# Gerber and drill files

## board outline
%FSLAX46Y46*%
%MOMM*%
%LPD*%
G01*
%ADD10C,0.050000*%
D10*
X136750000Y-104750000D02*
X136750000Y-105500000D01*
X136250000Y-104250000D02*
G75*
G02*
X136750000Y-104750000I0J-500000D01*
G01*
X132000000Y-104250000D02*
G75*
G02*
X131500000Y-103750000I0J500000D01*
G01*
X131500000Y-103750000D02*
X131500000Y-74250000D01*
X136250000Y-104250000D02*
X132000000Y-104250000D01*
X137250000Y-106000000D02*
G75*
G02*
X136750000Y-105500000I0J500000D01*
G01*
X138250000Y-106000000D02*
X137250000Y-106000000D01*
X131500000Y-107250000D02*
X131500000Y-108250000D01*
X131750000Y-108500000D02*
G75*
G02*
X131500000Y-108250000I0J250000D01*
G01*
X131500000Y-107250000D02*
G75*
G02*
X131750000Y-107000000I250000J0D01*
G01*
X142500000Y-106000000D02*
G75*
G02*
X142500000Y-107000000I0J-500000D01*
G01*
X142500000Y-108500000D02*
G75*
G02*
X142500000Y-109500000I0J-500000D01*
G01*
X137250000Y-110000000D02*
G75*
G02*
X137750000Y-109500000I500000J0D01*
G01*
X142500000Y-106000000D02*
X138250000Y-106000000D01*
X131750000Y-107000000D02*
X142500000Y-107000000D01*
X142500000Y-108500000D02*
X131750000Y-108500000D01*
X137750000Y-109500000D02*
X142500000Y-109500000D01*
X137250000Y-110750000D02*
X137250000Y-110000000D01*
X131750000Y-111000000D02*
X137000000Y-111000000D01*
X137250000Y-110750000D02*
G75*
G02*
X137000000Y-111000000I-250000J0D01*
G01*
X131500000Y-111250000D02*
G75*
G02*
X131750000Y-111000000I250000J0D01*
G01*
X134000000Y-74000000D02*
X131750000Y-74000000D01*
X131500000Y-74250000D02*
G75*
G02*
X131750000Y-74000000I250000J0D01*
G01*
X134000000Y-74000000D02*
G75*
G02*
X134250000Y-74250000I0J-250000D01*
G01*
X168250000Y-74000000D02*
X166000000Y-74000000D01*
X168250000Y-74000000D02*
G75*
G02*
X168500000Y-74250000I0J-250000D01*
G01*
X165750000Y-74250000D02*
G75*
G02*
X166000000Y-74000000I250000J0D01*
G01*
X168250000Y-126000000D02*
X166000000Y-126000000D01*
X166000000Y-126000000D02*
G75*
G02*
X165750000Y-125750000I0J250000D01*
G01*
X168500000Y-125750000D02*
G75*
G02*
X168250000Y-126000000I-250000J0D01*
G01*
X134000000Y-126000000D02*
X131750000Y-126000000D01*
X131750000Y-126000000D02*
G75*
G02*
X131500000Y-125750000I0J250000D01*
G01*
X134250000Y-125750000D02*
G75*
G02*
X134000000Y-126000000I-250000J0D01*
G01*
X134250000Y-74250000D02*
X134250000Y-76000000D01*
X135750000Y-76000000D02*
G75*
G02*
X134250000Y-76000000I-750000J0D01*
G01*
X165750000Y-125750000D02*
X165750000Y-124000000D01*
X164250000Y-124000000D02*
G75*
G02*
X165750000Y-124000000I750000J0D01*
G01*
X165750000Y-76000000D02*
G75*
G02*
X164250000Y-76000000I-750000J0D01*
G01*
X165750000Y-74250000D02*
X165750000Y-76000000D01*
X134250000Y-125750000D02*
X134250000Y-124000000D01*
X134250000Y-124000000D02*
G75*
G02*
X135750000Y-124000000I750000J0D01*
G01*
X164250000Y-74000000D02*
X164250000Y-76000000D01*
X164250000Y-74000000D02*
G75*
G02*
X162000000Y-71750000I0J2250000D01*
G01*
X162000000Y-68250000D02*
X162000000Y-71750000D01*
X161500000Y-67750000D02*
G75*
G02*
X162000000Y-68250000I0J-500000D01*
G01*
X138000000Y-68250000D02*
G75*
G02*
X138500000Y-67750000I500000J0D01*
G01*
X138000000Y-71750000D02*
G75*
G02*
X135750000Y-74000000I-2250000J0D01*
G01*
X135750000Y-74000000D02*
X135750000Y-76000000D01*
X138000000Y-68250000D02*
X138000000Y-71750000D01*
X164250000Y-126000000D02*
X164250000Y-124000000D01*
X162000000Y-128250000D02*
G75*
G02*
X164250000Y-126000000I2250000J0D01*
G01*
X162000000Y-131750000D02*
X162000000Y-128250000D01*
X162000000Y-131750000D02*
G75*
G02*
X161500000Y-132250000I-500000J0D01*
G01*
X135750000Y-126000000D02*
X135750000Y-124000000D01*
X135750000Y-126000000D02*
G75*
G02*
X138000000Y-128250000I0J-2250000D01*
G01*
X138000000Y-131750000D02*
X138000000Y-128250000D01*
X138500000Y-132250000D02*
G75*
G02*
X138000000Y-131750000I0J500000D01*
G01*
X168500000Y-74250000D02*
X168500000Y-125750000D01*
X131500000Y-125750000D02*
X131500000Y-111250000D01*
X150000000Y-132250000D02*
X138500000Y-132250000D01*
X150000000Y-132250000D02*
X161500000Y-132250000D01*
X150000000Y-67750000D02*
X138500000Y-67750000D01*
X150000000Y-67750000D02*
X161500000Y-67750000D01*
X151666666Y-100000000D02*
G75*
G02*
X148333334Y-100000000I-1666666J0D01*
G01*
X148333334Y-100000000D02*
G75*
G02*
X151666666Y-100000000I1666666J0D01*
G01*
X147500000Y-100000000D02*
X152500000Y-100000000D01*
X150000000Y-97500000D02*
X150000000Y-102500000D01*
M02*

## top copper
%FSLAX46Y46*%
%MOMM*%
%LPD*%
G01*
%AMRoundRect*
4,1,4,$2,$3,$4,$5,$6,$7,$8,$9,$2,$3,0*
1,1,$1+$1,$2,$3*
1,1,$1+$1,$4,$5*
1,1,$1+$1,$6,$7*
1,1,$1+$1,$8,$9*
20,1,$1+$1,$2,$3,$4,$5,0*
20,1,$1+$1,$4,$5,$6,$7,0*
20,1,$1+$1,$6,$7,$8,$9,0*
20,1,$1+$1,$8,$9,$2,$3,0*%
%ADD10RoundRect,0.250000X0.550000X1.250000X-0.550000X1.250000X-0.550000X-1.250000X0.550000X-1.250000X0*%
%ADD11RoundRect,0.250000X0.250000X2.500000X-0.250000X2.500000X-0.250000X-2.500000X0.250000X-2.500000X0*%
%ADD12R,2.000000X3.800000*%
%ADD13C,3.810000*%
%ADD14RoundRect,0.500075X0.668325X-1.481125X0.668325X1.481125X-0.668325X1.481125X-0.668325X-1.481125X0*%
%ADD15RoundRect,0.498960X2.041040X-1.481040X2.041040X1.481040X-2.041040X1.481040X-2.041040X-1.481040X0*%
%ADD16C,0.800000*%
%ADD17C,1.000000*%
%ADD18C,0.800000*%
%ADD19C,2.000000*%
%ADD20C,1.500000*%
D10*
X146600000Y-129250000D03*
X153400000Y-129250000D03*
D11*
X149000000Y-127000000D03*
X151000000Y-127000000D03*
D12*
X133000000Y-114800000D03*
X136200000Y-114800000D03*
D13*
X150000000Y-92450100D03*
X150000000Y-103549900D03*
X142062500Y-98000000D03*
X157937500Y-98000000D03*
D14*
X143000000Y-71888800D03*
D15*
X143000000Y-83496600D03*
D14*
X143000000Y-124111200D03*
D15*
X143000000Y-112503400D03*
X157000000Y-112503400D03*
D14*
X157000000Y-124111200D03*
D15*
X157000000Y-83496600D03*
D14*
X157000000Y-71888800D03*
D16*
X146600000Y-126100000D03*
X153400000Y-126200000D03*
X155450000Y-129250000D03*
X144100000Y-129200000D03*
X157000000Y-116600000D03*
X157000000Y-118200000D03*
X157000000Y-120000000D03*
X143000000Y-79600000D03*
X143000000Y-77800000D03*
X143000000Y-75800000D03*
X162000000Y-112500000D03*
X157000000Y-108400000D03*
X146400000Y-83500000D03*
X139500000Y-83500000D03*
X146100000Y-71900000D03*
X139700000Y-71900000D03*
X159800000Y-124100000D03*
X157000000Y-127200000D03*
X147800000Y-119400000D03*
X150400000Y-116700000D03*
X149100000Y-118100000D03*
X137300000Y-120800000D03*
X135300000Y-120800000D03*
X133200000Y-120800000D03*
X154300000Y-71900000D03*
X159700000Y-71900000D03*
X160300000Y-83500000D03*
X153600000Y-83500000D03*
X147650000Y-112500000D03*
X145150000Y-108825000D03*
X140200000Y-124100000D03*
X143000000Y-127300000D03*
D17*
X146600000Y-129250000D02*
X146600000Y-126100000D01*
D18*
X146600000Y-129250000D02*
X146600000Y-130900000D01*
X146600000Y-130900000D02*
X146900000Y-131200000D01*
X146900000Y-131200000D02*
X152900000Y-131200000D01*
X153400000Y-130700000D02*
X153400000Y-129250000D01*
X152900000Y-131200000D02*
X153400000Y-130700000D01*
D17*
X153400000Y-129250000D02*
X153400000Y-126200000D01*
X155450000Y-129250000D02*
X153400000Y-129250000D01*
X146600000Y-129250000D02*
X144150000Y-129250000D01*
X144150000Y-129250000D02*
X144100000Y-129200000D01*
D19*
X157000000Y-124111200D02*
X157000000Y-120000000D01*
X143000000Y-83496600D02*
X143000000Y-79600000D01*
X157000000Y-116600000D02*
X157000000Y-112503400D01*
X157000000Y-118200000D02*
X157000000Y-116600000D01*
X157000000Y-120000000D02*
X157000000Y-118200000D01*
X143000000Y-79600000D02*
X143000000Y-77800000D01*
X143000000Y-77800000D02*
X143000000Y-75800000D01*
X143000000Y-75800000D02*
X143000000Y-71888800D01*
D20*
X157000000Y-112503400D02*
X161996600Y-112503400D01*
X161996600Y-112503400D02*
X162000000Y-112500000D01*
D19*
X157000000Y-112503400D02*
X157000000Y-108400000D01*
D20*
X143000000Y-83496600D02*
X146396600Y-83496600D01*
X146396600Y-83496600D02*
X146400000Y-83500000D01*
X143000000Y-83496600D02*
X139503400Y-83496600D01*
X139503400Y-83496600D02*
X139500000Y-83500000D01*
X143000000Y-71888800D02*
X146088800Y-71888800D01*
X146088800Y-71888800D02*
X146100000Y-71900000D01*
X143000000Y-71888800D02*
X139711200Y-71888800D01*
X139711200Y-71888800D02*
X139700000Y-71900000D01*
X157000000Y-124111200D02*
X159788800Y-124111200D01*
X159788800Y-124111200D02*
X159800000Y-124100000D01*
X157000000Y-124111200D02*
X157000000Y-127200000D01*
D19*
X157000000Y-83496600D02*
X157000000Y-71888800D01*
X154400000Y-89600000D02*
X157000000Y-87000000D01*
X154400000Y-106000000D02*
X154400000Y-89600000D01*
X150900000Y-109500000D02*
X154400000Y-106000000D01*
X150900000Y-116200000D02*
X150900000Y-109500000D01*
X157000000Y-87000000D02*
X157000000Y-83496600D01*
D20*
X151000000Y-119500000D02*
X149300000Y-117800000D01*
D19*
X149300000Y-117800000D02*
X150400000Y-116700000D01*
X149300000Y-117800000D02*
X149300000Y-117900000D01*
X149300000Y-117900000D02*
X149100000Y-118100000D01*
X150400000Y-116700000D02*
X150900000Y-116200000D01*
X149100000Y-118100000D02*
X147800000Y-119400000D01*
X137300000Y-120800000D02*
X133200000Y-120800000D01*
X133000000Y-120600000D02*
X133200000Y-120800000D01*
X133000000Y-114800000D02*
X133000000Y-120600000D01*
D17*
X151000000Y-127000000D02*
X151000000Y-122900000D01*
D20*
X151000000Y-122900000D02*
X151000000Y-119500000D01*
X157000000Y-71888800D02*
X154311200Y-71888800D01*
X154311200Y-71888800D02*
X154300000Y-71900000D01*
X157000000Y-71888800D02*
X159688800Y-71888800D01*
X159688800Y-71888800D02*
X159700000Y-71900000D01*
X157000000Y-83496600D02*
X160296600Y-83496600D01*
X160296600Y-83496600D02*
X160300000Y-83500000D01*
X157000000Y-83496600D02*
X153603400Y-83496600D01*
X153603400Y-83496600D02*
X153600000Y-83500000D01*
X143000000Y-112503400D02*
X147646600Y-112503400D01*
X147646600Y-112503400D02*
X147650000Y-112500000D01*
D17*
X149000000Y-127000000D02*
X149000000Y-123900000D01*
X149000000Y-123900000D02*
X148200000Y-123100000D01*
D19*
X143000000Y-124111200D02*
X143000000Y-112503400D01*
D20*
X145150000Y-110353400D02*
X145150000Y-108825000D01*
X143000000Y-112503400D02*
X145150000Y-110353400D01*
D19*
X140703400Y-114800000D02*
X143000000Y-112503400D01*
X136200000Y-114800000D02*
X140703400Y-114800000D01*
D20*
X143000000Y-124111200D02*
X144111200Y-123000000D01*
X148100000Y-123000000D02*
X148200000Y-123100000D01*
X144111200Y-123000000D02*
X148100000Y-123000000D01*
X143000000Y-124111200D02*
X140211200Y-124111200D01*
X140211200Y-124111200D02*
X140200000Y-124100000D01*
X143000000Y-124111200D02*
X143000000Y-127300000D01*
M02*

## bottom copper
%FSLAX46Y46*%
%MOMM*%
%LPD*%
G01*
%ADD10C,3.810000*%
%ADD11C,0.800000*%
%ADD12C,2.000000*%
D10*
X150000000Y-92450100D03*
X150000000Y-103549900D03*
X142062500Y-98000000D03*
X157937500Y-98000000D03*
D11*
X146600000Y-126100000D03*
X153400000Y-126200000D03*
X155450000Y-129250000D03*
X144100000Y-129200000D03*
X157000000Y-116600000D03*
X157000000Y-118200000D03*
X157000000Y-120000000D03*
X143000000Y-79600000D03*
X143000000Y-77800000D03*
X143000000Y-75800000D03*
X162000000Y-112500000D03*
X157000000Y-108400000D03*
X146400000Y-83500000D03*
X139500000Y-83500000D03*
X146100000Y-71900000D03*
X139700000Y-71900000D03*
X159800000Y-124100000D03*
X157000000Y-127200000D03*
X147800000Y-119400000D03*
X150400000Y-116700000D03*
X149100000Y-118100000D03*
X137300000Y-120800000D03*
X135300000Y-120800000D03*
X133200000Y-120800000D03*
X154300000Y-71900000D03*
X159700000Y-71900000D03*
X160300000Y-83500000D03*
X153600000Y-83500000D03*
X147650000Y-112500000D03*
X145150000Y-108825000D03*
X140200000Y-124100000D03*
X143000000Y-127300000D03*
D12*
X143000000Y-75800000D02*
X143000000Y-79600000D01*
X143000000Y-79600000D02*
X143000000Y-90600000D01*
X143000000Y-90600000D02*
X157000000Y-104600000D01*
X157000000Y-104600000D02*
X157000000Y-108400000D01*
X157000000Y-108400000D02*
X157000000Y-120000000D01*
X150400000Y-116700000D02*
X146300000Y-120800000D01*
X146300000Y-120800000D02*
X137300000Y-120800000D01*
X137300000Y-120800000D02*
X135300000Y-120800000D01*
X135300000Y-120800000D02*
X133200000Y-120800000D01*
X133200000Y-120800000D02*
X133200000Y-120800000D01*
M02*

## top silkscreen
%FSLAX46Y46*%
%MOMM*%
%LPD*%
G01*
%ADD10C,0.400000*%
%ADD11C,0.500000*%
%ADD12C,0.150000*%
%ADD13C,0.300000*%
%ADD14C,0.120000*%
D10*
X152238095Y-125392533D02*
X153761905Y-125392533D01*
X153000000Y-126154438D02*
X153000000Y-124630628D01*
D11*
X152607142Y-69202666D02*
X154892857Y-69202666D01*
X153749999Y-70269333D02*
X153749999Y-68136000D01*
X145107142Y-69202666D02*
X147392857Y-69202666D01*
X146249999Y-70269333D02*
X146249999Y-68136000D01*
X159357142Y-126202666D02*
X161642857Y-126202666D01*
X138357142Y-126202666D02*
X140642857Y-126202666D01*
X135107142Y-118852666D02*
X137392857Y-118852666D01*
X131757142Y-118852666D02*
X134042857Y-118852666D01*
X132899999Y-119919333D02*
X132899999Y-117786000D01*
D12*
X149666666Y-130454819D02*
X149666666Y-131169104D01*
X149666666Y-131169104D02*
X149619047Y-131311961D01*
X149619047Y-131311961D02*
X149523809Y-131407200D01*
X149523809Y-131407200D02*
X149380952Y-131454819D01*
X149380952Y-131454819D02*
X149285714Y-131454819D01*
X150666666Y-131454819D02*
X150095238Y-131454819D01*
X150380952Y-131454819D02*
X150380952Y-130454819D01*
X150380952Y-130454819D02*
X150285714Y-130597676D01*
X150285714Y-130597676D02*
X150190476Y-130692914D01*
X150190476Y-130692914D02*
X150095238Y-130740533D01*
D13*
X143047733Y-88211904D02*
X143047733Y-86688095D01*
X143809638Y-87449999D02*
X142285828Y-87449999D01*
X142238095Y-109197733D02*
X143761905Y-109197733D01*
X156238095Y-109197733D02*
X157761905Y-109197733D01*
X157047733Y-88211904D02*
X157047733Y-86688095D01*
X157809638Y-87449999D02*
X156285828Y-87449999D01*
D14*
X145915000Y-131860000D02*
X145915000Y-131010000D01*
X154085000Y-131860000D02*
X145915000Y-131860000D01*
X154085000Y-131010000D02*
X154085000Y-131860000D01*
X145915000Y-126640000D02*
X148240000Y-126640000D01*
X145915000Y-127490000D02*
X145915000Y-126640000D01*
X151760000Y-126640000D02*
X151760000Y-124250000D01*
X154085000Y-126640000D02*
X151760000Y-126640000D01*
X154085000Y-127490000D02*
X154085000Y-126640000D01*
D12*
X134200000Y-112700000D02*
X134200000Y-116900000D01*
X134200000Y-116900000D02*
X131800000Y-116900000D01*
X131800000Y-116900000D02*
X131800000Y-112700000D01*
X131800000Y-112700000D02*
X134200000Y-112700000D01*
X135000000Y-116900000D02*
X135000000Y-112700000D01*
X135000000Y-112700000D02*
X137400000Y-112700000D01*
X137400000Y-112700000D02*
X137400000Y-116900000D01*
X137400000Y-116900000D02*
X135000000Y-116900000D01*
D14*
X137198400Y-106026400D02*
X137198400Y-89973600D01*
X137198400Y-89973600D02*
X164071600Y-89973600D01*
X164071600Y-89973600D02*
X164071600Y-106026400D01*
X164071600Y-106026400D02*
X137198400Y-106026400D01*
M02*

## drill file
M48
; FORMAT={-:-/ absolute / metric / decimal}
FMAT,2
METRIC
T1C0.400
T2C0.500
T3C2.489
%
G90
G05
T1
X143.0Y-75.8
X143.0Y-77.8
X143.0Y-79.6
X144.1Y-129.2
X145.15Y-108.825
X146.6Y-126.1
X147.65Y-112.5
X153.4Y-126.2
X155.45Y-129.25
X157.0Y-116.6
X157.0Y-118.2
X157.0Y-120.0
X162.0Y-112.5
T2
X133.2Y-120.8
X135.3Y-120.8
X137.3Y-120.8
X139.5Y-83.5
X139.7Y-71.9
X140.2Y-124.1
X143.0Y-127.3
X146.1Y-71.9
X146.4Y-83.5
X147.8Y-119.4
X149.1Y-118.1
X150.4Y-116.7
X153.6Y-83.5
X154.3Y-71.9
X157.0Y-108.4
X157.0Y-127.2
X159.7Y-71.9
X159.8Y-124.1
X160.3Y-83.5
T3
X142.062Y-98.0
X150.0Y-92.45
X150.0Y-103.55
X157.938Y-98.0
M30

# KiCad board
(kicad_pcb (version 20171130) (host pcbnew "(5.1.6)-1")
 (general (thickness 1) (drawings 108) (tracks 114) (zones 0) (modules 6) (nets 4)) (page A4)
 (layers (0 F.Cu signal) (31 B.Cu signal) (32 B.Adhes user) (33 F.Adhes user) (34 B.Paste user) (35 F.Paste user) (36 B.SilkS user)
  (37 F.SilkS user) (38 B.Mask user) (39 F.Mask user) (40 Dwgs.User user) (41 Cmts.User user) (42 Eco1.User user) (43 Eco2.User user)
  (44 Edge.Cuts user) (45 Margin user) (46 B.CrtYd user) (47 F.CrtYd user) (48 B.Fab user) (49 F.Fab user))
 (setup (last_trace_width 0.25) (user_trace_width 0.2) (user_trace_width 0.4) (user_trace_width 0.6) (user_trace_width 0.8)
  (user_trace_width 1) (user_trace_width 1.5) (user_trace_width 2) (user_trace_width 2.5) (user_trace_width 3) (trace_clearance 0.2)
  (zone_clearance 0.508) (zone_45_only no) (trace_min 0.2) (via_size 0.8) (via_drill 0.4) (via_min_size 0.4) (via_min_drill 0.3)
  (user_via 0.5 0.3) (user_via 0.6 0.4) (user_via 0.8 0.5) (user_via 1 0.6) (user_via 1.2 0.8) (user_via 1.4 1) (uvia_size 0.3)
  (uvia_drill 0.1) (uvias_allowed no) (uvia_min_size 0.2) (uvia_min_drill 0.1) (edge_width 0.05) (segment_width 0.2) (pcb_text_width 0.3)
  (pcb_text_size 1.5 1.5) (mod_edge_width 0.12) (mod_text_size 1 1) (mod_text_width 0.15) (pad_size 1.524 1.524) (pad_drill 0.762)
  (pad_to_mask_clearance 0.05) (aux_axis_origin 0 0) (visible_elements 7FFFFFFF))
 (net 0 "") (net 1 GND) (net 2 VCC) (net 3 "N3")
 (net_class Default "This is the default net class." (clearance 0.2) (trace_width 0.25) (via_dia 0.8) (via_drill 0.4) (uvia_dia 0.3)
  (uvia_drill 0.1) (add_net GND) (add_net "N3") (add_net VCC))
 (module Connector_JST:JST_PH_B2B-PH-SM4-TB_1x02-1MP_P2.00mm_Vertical (layer F.Cu) (at 150 127.5 180)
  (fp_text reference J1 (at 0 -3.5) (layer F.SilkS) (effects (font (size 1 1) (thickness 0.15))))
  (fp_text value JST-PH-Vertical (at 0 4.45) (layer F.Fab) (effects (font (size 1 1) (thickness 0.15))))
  (fp_line (start 4.085 -4.36) (end 4.085 -3.51) (layer F.SilkS) (width 0.12))
  (fp_line (start -4.085 -4.36) (end 4.085 -4.36) (layer F.SilkS) (width 0.12))
  (fp_line (start -4.085 -3.51) (end -4.085 -4.36) (layer F.SilkS) (width 0.12))
  (fp_line (start 4.085 0.86) (end 1.76 0.86) (layer F.SilkS) (width 0.12))
  (fp_line (start 4.085 0.01) (end 4.085 0.86) (layer F.SilkS) (width 0.12))
  (fp_line (start -1.76 0.86) (end -1.76 3.25) (layer F.SilkS) (width 0.12))
  (fp_line (start -4.085 0.86) (end -1.76 0.86) (layer F.SilkS) (width 0.12))
  (fp_line (start -4.085 0.01) (end -4.085 0.86) (layer F.SilkS) (width 0.12))
  (pad MP smd roundrect (at 3.4 -1.75 180) (size 1.6 3) (layers F.Cu F.Paste F.Mask) (roundrect_rratio 0.15625))
  (pad MP smd roundrect (at -3.4 -1.75 180) (size 1.6 3) (layers F.Cu F.Paste F.Mask) (roundrect_rratio 0.15625))
  (pad 2 smd roundrect (at 1 0.5 180) (size 1 5.5) (layers F.Cu F.Paste F.Mask) (roundrect_rratio 0.25) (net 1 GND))
  (pad 1 smd roundrect (at -1 0.5 180) (size 1 5.5) (layers F.Cu F.Paste F.Mask) (roundrect_rratio 0.25) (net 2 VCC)))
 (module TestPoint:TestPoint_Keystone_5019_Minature (layer F.Cu) (at 133 114.8 270)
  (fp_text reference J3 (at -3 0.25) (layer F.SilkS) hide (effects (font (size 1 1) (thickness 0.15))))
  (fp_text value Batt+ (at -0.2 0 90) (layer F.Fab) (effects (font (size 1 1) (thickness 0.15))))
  (fp_line (start -2.1 -1.2) (end 2.1 -1.2) (layer F.SilkS) (width 0.15))
  (fp_line (start 2.1 -1.2) (end 2.1 1.2) (layer F.SilkS) (width 0.15))
  (fp_line (start 2.1 1.2) (end -2.1 1.2) (layer F.SilkS) (width 0.15))
  (fp_line (start -2.1 1.2) (end -2.1 -1.2) (layer F.SilkS) (width 0.15))
  (pad 1 smd rect (at 0 0 270) (size 3.8 2) (layers F.Cu F.Paste F.Mask) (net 2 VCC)))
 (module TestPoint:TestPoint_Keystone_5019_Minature (layer F.Cu) (at 136.2 114.8 90)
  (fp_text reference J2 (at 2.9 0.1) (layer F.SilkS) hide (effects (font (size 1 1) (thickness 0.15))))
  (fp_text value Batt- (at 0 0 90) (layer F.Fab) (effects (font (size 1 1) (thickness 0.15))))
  (fp_line (start -2.1 -1.2) (end 2.1 -1.2) (layer F.SilkS) (width 0.15))
  (fp_line (start 2.1 -1.2) (end 2.1 1.2) (layer F.SilkS) (width 0.15))
  (fp_line (start 2.1 1.2) (end -2.1 1.2) (layer F.SilkS) (width 0.15))
  (fp_line (start -2.1 1.2) (end -2.1 -1.2) (layer F.SilkS) (width 0.15))
  (pad 1 smd rect (at 0 0 90) (size 3.8 2) (layers F.Cu F.Paste F.Mask) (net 1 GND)))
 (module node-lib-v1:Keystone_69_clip (layer F.Cu) (at 150 98 180)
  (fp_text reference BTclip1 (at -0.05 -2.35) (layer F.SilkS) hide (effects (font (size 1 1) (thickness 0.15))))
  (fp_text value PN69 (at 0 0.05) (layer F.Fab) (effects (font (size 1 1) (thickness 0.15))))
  (fp_line (start 12.8016 -8.0264) (end 12.8016 8.0264) (layer F.SilkS) (width 0.12))
  (fp_line (start 12.8016 8.0264) (end -14.0716 8.0264) (layer F.SilkS) (width 0.12))
  (fp_line (start -14.0716 8.0264) (end -14.0716 -8.0264) (layer F.SilkS) (width 0.12))
  (fp_line (start -14.0716 -8.0264) (end 12.8016 -8.0264) (layer F.SilkS) (width 0.12))
  (pad 2 smd circle (at 7.9375 0 180) (size 3.81 3.81) (layers F.Paste F.Mask))
  (pad 2 smd circle (at -7.9375 0 180) (size 3.81 3.81) (layers F.Paste F.Mask))
  (pad 2 smd circle (at 0 -5.5499 180) (size 3.81 3.81) (layers F.Paste F.Mask))
  (pad 2 smd circle (at 0 5.5499 180) (size 3.81 3.81) (layers F.Paste F.Mask))
  (pad 1 thru_hole circle (at 0 5.5499 180) (size 3.81 3.81) (drill 2.4892) (layers *.Cu *.Mask))
  (pad 1 thru_hole circle (at 0 -5.5499 180) (size 3.81 3.81) (drill 2.4892) (layers *.Cu *.Mask))
  (pad 1 thru_hole circle (at 7.9375 0 180) (size 3.81 3.81) (drill 2.4892) (layers *.Cu *.Mask))
  (pad 1 thru_hole circle (at -7.9375 0 180) (size 3.81 3.81) (drill 2.4892) (layers *.Cu *.Mask F.Paste)))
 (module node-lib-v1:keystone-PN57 (layer F.Cu) (at 143 98 90)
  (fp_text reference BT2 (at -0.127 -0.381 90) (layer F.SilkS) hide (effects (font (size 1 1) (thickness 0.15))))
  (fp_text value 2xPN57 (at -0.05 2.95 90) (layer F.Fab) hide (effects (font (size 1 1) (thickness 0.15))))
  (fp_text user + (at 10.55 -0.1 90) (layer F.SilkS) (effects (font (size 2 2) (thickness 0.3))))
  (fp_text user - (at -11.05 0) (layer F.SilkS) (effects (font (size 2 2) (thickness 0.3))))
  (pad 1 smd roundrect (at 26.1112 0 90) (size 3.9624 2.3368) (layers F.Cu F.Paste F.Mask) (roundrect_rratio 0.214) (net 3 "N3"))
  (pad 1 smd roundrect (at 14.5034 0 90) (size 3.96 5.08) (layers F.Cu F.Paste F.Mask) (roundrect_rratio 0.126) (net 3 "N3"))
  (pad 2 smd roundrect (at -26.1112 0 90) (size 3.9624 2.3368) (layers F.Cu F.Paste F.Mask) (roundrect_rratio 0.214) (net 1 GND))
  (pad 2 smd roundrect (at -14.5034 0 90) (size 3.96 5.08) (layers F.Cu F.Paste F.Mask) (roundrect_rratio 0.126) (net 1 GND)))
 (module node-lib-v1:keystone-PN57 (layer F.Cu) (at 157 98 90)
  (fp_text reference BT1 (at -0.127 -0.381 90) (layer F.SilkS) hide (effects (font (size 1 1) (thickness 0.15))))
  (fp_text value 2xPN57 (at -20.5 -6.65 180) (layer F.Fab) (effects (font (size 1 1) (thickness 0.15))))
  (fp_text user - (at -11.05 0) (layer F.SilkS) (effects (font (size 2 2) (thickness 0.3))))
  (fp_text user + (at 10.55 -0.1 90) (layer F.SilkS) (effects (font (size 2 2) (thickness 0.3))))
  (pad 2 smd roundrect (at -14.5034 0 90) (size 3.96 5.08) (layers F.Cu F.Paste F.Mask) (roundrect_rratio 0.126) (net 3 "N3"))
  (pad 2 smd roundrect (at -26.1112 0 90) (size 3.9624 2.3368) (layers F.Cu F.Paste F.Mask) (roundrect_rratio 0.214) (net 3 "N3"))
  (pad 1 smd roundrect (at 14.5034 0 90) (size 3.96 5.08) (layers F.Cu F.Paste F.Mask) (roundrect_rratio 0.126) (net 2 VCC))
  (pad 1 smd roundrect (at 26.1112 0 90) (size 3.9624 2.3368) (layers F.Cu F.Paste F.Mask) (roundrect_rratio 0.214) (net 2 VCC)))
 (gr_line (start 136.75 104.75) (end 136.75 105.5) (layer Edge.Cuts) (width 0.05))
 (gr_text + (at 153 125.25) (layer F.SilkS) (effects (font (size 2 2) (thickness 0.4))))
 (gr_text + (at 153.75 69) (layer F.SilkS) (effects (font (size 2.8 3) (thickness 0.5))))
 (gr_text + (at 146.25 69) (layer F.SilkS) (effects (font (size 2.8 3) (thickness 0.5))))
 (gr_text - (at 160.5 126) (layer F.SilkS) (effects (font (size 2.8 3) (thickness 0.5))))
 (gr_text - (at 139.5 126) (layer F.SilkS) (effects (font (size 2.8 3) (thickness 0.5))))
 (gr_arc (start 136.25 104.75) (end 136.75 104.75) (angle -90) (layer Edge.Cuts) (width 0.05))
 (gr_arc (start 132 103.75) (end 131.5 103.75) (angle -90) (layer Edge.Cuts) (width 0.05))
 (gr_line (start 131.5 103.75) (end 131.5 74.25) (layer Edge.Cuts) (width 0.05))
 (gr_line (start 136.25 104.25) (end 132 104.25) (layer Edge.Cuts) (width 0.05))
 (gr_arc (start 137.25 105.5) (end 136.75 105.5) (angle -90) (layer Edge.Cuts) (width 0.05))
 (gr_line (start 138.25 106) (end 137.25 106) (layer Edge.Cuts) (width 0.05))
 (gr_line (start 131.5 107.25) (end 131.5 108.25) (layer Edge.Cuts) (width 0.05))
 (gr_arc (start 131.75 108.25) (end 131.5 108.25) (angle -90) (layer Edge.Cuts) (width 0.05))
 (gr_arc (start 131.75 107.25) (end 131.75 107) (angle -90) (layer Edge.Cuts) (width 0.05))
 (gr_arc (start 142.5 106.5) (end 142.5 107) (angle -180) (layer Edge.Cuts) (width 0.05))
 (gr_arc (start 142.5 109) (end 142.5 109.5) (angle -180) (layer Edge.Cuts) (width 0.05))
 (gr_arc (start 137.75 110) (end 137.75 109.5) (angle -90) (layer Edge.Cuts) (width 0.05))
 (gr_line (start 142.5 106) (end 138.25 106) (layer Edge.Cuts) (width 0.05))
 (gr_line (start 131.75 107) (end 142.5 107) (layer Edge.Cuts) (width 0.05))
 (gr_line (start 142.5 108.5) (end 131.75 108.5) (layer Edge.Cuts) (width 0.05))
 (gr_line (start 137.75 109.5) (end 142.5 109.5) (layer Edge.Cuts) (width 0.05))
 (gr_line (start 137.25 110.75) (end 137.25 110) (layer Edge.Cuts) (width 0.05))
 (gr_line (start 131.75 111) (end 137 111) (layer Edge.Cuts) (width 0.05))
 (gr_arc (start 137 110.75) (end 137 111) (angle -90) (layer Edge.Cuts) (width 0.05))
 (gr_arc (start 131.75 111.25) (end 131.75 111) (angle -90) (layer Edge.Cuts) (width 0.05))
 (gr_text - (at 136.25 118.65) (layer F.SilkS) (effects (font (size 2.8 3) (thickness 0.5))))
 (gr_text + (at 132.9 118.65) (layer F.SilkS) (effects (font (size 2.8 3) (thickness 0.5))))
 (gr_line (start 134 74) (end 131.75 74) (layer Edge.Cuts) (width 0.05))
 (gr_arc (start 131.75 74.25) (end 131.75 74) (angle -90) (layer Edge.Cuts) (width 0.05))
 (gr_arc (start 134 74.25) (end 134.25 74.25) (angle -90) (layer Edge.Cuts) (width 0.05))
 (gr_line (start 168.25 74) (end 166 74) (layer Edge.Cuts) (width 0.05))
 (gr_arc (start 168.25 74.25) (end 168.5 74.25) (angle -90) (layer Edge.Cuts) (width 0.05))
 (gr_arc (start 166 74.25) (end 166 74) (angle -90) (layer Edge.Cuts) (width 0.05))
 (gr_line (start 168.25 126) (end 166 126) (layer Edge.Cuts) (width 0.05))
 (gr_arc (start 166 125.75) (end 165.75 125.75) (angle -90) (layer Edge.Cuts) (width 0.05))
 (gr_arc (start 168.25 125.75) (end 168.25 126) (angle -90) (layer Edge.Cuts) (width 0.05))
 (gr_line (start 134 126) (end 131.75 126) (layer Edge.Cuts) (width 0.05))
 (gr_arc (start 131.75 125.75) (end 131.5 125.75) (angle -90) (layer Edge.Cuts) (width 0.05))
 (gr_arc (start 134 125.75) (end 134 126) (angle -90) (layer Edge.Cuts) (width 0.05))
 (gr_line (start 134.25 74.25) (end 134.25 76) (layer Edge.Cuts) (width 0.05))
 (gr_arc (start 135 76) (end 134.25 76) (angle -180) (layer Edge.Cuts) (width 0.05))
 (gr_line (start 165.75 125.75) (end 165.75 124) (layer Edge.Cuts) (width 0.05))
 (gr_arc (start 165 124) (end 165.75 124) (angle -180) (layer Edge.Cuts) (width 0.05))
 (gr_arc (start 165 76) (end 164.25 76) (angle -180) (layer Edge.Cuts) (width 0.05))
 (gr_line (start 165.75 74.25) (end 165.75 76) (layer Edge.Cuts) (width 0.05))
 (gr_line (start 134.25 125.75) (end 134.25 124) (layer Edge.Cuts) (width 0.05))
 (gr_arc (start 135 124) (end 135.75 124) (angle -180) (layer Edge.Cuts) (width 0.05))
 (gr_line (start 164.25 74) (end 164.25 76) (layer Edge.Cuts) (width 0.05))
 (gr_arc (start 164.25 71.75) (end 162 71.75) (angle -90) (layer Edge.Cuts) (width 0.05))
 (gr_line (start 162 68.25) (end 162 71.75) (layer Edge.Cuts) (width 0.05))
 (gr_arc (start 161.5 68.25) (end 162 68.25) (angle -90) (layer Edge.Cuts) (width 0.05))
 (gr_arc (start 138.5 68.25) (end 138.5 67.75) (angle -90) (layer Edge.Cuts) (width 0.05))
 (gr_arc (start 135.75 71.75) (end 135.75 74) (angle -90) (layer Edge.Cuts) (width 0.05))
 (gr_line (start 135.75 74) (end 135.75 76) (layer Edge.Cuts) (width 0.05))
 (gr_line (start 138 68.25) (end 138 71.75) (layer Edge.Cuts) (width 0.05))
 (gr_line (start 164.25 126) (end 164.25 124) (layer Edge.Cuts) (width 0.05))
 (gr_arc (start 164.25 128.25) (end 164.25 126) (angle -90) (layer Edge.Cuts) (width 0.05))
 (gr_line (start 162 131.75) (end 162 128.25) (layer Edge.Cuts) (width 0.05))
 (gr_arc (start 161.5 131.75) (end 161.5 132.25) (angle -90) (layer Edge.Cuts) (width 0.05))
 (gr_line (start 135.75 126) (end 135.75 124) (layer Edge.Cuts) (width 0.05))
 (gr_arc (start 135.75 128.25) (end 138 128.25) (angle -90) (layer Edge.Cuts) (width 0.05))
 (gr_line (start 138 131.75) (end 138 128.25) (layer Edge.Cuts) (width 0.05))
 (gr_arc (start 138.5 131.75) (end 138 131.75) (angle -90) (layer Edge.Cuts) (width 0.05))
 (gr_line (start 168.5 74.25) (end 168.5 125.75) (layer Edge.Cuts) (width 0.05))
 (gr_line (start 131.5 125.75) (end 131.5 111.25) (layer Edge.Cuts) (width 0.05))
 (gr_line (start 150 132.25) (end 138.5 132.25) (layer Edge.Cuts) (width 0.05))
 (gr_line (start 150 132.25) (end 161.5 132.25) (layer Edge.Cuts) (width 0.05))
 (gr_line (start 150 67.75) (end 138.5 67.75) (layer Edge.Cuts) (width 0.05))
 (gr_line (start 150 67.75) (end 161.5 67.75) (layer Edge.Cuts) (width 0.05))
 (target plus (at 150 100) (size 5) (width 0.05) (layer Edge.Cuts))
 (via (at 146.6 126.1) (size 0.8) (drill 0.4) (layers F.Cu B.Cu) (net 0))
 (segment (start 146.6 129.25) (end 146.6 126.1) (width 1) (layer F.Cu) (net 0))
 (segment (start 146.6 129.25) (end 146.6 130.9) (width 0.8) (layer F.Cu) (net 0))
 (segment (start 146.6 130.9) (end 146.9 131.2) (width 0.8) (layer F.Cu) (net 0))
 (segment (start 146.9 131.2) (end 152.9 131.2) (width 0.8) (layer F.Cu) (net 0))
 (segment (start 153.4 130.7) (end 153.4 129.25) (width 0.8) (layer F.Cu) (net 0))
 (segment (start 152.9 131.2) (end 153.4 130.7) (width 0.8) (layer F.Cu) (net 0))
 (via (at 153.4 126.2) (size 0.8) (drill 0.4) (layers F.Cu B.Cu) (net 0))
 (segment (start 153.4 129.25) (end 153.4 126.2) (width 1) (layer F.Cu) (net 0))
 (segment (start 155.45 129.25) (end 153.4 129.25) (width 1) (layer F.Cu) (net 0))
 (via (at 155.45 129.25) (size 0.8) (drill 0.4) (layers F.Cu B.Cu) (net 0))
 (segment (start 146.6 129.25) (end 144.15 129.25) (width 1) (layer F.Cu) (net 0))
 (via (at 144.1 129.2) (size 0.8) (drill 0.4) (layers F.Cu B.Cu) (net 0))
 (segment (start 144.15 129.25) (end 144.1 129.2) (width 1) (layer F.Cu) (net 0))
 (segment (start 157 124.1112) (end 157 120) (width 2) (layer F.Cu) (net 3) (status 30))
 (segment (start 143 83.4966) (end 143 79.6) (width 2) (layer F.Cu) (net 3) (status 30))
 (segment (start 157 116.6) (end 157 112.5034) (width 2) (layer F.Cu) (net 3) (status 30))
 (via (at 157 116.6) (size 0.8) (drill 0.4) (layers F.Cu B.Cu) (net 3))
 (segment (start 157 118.2) (end 157 116.6) (width 2) (layer F.Cu) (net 3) (status 30))
 (via (at 157 118.2) (size 0.8) (drill 0.4) (layers F.Cu B.Cu) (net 3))
 (segment (start 157 120) (end 157 118.2) (width 2) (layer F.Cu) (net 3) (status 30))
 (via (at 157 120) (size 0.8) (drill 0.4) (layers F.Cu B.Cu) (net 3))
 (segment (start 143 79.6) (end 143 77.8) (width 2) (layer F.Cu) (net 3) (status 30))
 (via (at 143 79.6) (size 0.8) (drill 0.4) (layers F.Cu B.Cu) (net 3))
 (segment (start 143 77.8) (end 143 75.8) (width 2) (layer F.Cu) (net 3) (status 30))
 (via (at 143 77.8) (size 0.8) (drill 0.4) (layers F.Cu B.Cu) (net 3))
 (segment (start 143 75.8) (end 143 71.8888) (width 2) (layer F.Cu) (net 3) (status 30))
 (via (at 143 75.8) (size 0.8) (drill 0.4) (layers F.Cu B.Cu) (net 3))
 (segment (start 143 75.8) (end 143 79.6) (width 2) (layer B.Cu) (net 3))
 (segment (start 143 79.6) (end 143 90.6) (width 2) (layer B.Cu) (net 3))
 (segment (start 143 90.6) (end 157 104.6) (width 2) (layer B.Cu) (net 3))
 (via (at 162 112.5) (size 0.8) (drill 0.4) (layers F.Cu B.Cu) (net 3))
 (segment (start 157 112.5034) (end 161.9966 112.5034) (width 1.5) (layer F.Cu) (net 3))
 (segment (start 161.9966 112.5034) (end 162 112.5) (width 1.5) (layer F.Cu) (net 3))
 (segment (start 157 112.5034) (end 157 108.4) (width 2) (layer F.Cu) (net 3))
 (via (at 157 108.4) (size 0.8) (drill 0.5) (layers F.Cu B.Cu) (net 3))
 (segment (start 157 104.6) (end 157 108.4) (width 2) (layer B.Cu) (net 3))
 (segment (start 157 108.4) (end 157 120) (width 2) (layer B.Cu) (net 3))
 (via (at 146.4 83.5) (size 0.8) (drill 0.5) (layers F.Cu B.Cu) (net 3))
 (segment (start 143 83.4966) (end 146.3966 83.4966) (width 1.5) (layer F.Cu) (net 3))
 (segment (start 146.3966 83.4966) (end 146.4 83.5) (width 1.5) (layer F.Cu) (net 3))
 (via (at 139.5 83.5) (size 0.8) (drill 0.5) (layers F.Cu B.Cu) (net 3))
 (segment (start 143 83.4966) (end 139.5034 83.4966) (width 1.5) (layer F.Cu) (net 3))
 (segment (start 139.5034 83.4966) (end 139.5 83.5) (width 1.5) (layer F.Cu) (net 3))
 (via (at 146.1 71.9) (size 0.8) (drill 0.5) (layers F.Cu B.Cu) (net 3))
 (segment (start 143 71.8888) (end 146.0888 71.8888) (width 1.5) (layer F.Cu) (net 3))
 (segment (start 146.0888 71.8888) (end 146.1 71.9) (width 1.5) (layer F.Cu) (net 3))
 (via (at 139.7 71.9) (size 0.8) (drill 0.5) (layers F.Cu B.Cu) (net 3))
 (segment (start 143 71.8888) (end 139.7112 71.8888) (width 1.5) (layer F.Cu) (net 3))
 (segment (start 139.7112 71.8888) (end 139.7 71.9) (width 1.5) (layer F.Cu) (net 3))
 (via (at 159.8 124.1) (size 0.8) (drill 0.5) (layers F.Cu B.Cu) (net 3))
 (segment (start 157 124.1112) (end 159.7888 124.1112) (width 1.5) (layer F.Cu) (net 3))
 (segment (start 159.7888 124.1112) (end 159.8 124.1) (width 1.5) (layer F.Cu) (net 3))
 (via (at 157 127.2) (size 0.8) (drill 0.5) (layers F.Cu B.Cu) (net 3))
 (segment (start 157 124.1112) (end 157 127.2) (width 1.5) (layer F.Cu) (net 3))
 (segment (start 157 83.4966) (end 157 71.8888) (width 2) (layer F.Cu) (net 2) (status 30))
 (segment (start 154.4 89.6) (end 157 87) (width 2) (layer F.Cu) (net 2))
 (segment (start 154.4 106) (end 154.4 89.6) (width 2) (layer F.Cu) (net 2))
 (segment (start 150.9 109.5) (end 154.4 106) (width 2) (layer F.Cu) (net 2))
 (segment (start 150.9 116.2) (end 150.9 109.5) (width 2) (layer F.Cu) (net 2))
 (segment (start 157 87) (end 157 83.4966) (width 2) (layer F.Cu) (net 2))
 (segment (start 151 119.5) (end 149.3 117.8) (width 1.5) (layer F.Cu) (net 2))
 (segment (start 149.3 117.8) (end 150.4 116.7) (width 2) (layer F.Cu) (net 2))
 (via (at 147.8 119.4) (size 0.8) (drill 0.5) (layers F.Cu B.Cu) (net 2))
 (segment (start 149.3 117.8) (end 149.3 117.9) (width 2) (layer F.Cu) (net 2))
 (segment (start 149.3 117.9) (end 149.1 118.1) (width 2) (layer F.Cu) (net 2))
 (segment (start 150.4 116.7) (end 150.9 116.2) (width 2) (layer F.Cu) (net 2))
 (via (at 150.4 116.7) (size 0.8) (drill 0.5) (layers F.Cu B.Cu) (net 2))
 (segment (start 149.1 118.1) (end 147.8 119.4) (width 2) (layer F.Cu) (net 2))
 (via (at 149.1 118.1) (size 0.8) (drill 0.5) (layers F.Cu B.Cu) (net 2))
 (segment (start 150.4 116.7) (end 146.3 120.8) (width 2) (layer B.Cu) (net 2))
 (segment (start 146.3 120.8) (end 137.3 120.8) (width 2) (layer B.Cu) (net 2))
 (segment (start 137.3 120.8) (end 135.3 120.8) (width 2) (layer B.Cu) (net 2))
 (via (at 137.3 120.8) (size 0.8) (drill 0.5) (layers F.Cu B.Cu) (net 2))
 (segment (start 135.3 120.8) (end 133.2 120.8) (width 2) (layer B.Cu) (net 2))
 (via (at 135.3 120.8) (size 0.8) (drill 0.5) (layers F.Cu B.Cu) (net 2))
 (segment (start 133.2 120.8) (end 133.2 120.8) (width 2) (layer B.Cu) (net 2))
 (via (at 133.2 120.8) (size 0.8) (drill 0.5) (layers F.Cu B.Cu) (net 2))
 (segment (start 137.3 120.8) (end 133.2 120.8) (width 2) (layer F.Cu) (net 2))
 (segment (start 133 120.6) (end 133.2 120.8) (width 2) (layer F.Cu) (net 2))
 (segment (start 133 114.8) (end 133 120.6) (width 2) (layer F.Cu) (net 2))
 (segment (start 151 127) (end 151 122.9) (width 1) (layer F.Cu) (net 2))
 (segment (start 151 122.9) (end 151 119.5) (width 1.5) (layer F.Cu) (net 2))
 (via (at 154.3 71.9) (size 0.8) (drill 0.5) (layers F.Cu B.Cu) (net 2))
 (segment (start 157 71.8888) (end 154.3112 71.8888) (width 1.5) (layer F.Cu) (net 2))
 (segment (start 154.3112 71.8888) (end 154.3 71.9) (width 1.5) (layer F.Cu) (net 2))
 (segment (start 157 71.8888) (end 159.6888 71.8888) (width 1.5) (layer F.Cu) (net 2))
 (via (at 159.7 71.9) (size 0.8) (drill 0.5) (layers F.Cu B.Cu) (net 2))
 (segment (start 159.6888 71.8888) (end 159.7 71.9) (width 1.5) (layer F.Cu) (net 2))
 (via (at 160.3 83.5) (size 0.8) (drill 0.5) (layers F.Cu B.Cu) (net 2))
 (segment (start 157 83.4966) (end 160.2966 83.4966) (width 1.5) (layer F.Cu) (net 2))
 (segment (start 160.2966 83.4966) (end 160.3 83.5) (width 1.5) (layer F.Cu) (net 2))
 (via (at 153.6 83.5) (size 0.8) (drill 0.5) (layers F.Cu B.Cu) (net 2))
 (segment (start 157 83.4966) (end 153.6034 83.4966) (width 1.5) (layer F.Cu) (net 2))
 (segment (start 153.6034 83.4966) (end 153.6 83.5) (width 1.5) (layer F.Cu) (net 2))
 (via (at 147.65 112.5) (size 0.8) (drill 0.4) (layers F.Cu B.Cu) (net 1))
 (segment (start 143 112.5034) (end 147.6466 112.5034) (width 1.5) (layer F.Cu) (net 1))
 (segment (start 147.6466 112.5034) (end 147.65 112.5) (width 1.5) (layer F.Cu) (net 1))
 (via (at 145.15 108.825) (size 0.8) (drill 0.4) (layers F.Cu B.Cu) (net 1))
 (segment (start 149 127) (end 149 123.9) (width 1) (layer F.Cu) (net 1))
 (segment (start 149 123.9) (end 148.2 123.1) (width 1) (layer F.Cu) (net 1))
 (segment (start 143 124.1112) (end 143 112.5034) (width 2) (layer F.Cu) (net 1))
 (segment (start 145.15 110.3534) (end 145.15 108.825) (width 1.5) (layer F.Cu) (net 1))
 (segment (start 143 112.5034) (end 145.15 110.3534) (width 1.5) (layer F.Cu) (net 1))
 (segment (start 140.7034 114.8) (end 143 112.5034) (width 2) (layer F.Cu) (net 1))
 (segment (start 136.2 114.8) (end 140.7034 114.8) (width 2) (layer F.Cu) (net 1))
 (segment (start 143 124.1112) (end 144.1112 123) (width 1.5) (layer F.Cu) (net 1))
 (segment (start 148.1 123) (end 148.2 123.1) (width 1.5) (layer F.Cu) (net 1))
 (segment (start 144.1112 123) (end 148.1 123) (width 1.5) (layer F.Cu) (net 1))
 (via (at 140.2 124.1) (size 0.8) (drill 0.5) (layers F.Cu B.Cu) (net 1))
 (segment (start 143 124.1112) (end 140.2112 124.1112) (width 1.5) (layer F.Cu) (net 1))
 (segment (start 140.2112 124.1112) (end 140.2 124.1) (width 1.5) (layer F.Cu) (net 1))
 (via (at 143 127.3) (size 0.8) (drill 0.5) (layers F.Cu B.Cu) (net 1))
 (segment (start 143 124.1112) (end 143 127.3) (width 1.5) (layer F.Cu) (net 1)))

